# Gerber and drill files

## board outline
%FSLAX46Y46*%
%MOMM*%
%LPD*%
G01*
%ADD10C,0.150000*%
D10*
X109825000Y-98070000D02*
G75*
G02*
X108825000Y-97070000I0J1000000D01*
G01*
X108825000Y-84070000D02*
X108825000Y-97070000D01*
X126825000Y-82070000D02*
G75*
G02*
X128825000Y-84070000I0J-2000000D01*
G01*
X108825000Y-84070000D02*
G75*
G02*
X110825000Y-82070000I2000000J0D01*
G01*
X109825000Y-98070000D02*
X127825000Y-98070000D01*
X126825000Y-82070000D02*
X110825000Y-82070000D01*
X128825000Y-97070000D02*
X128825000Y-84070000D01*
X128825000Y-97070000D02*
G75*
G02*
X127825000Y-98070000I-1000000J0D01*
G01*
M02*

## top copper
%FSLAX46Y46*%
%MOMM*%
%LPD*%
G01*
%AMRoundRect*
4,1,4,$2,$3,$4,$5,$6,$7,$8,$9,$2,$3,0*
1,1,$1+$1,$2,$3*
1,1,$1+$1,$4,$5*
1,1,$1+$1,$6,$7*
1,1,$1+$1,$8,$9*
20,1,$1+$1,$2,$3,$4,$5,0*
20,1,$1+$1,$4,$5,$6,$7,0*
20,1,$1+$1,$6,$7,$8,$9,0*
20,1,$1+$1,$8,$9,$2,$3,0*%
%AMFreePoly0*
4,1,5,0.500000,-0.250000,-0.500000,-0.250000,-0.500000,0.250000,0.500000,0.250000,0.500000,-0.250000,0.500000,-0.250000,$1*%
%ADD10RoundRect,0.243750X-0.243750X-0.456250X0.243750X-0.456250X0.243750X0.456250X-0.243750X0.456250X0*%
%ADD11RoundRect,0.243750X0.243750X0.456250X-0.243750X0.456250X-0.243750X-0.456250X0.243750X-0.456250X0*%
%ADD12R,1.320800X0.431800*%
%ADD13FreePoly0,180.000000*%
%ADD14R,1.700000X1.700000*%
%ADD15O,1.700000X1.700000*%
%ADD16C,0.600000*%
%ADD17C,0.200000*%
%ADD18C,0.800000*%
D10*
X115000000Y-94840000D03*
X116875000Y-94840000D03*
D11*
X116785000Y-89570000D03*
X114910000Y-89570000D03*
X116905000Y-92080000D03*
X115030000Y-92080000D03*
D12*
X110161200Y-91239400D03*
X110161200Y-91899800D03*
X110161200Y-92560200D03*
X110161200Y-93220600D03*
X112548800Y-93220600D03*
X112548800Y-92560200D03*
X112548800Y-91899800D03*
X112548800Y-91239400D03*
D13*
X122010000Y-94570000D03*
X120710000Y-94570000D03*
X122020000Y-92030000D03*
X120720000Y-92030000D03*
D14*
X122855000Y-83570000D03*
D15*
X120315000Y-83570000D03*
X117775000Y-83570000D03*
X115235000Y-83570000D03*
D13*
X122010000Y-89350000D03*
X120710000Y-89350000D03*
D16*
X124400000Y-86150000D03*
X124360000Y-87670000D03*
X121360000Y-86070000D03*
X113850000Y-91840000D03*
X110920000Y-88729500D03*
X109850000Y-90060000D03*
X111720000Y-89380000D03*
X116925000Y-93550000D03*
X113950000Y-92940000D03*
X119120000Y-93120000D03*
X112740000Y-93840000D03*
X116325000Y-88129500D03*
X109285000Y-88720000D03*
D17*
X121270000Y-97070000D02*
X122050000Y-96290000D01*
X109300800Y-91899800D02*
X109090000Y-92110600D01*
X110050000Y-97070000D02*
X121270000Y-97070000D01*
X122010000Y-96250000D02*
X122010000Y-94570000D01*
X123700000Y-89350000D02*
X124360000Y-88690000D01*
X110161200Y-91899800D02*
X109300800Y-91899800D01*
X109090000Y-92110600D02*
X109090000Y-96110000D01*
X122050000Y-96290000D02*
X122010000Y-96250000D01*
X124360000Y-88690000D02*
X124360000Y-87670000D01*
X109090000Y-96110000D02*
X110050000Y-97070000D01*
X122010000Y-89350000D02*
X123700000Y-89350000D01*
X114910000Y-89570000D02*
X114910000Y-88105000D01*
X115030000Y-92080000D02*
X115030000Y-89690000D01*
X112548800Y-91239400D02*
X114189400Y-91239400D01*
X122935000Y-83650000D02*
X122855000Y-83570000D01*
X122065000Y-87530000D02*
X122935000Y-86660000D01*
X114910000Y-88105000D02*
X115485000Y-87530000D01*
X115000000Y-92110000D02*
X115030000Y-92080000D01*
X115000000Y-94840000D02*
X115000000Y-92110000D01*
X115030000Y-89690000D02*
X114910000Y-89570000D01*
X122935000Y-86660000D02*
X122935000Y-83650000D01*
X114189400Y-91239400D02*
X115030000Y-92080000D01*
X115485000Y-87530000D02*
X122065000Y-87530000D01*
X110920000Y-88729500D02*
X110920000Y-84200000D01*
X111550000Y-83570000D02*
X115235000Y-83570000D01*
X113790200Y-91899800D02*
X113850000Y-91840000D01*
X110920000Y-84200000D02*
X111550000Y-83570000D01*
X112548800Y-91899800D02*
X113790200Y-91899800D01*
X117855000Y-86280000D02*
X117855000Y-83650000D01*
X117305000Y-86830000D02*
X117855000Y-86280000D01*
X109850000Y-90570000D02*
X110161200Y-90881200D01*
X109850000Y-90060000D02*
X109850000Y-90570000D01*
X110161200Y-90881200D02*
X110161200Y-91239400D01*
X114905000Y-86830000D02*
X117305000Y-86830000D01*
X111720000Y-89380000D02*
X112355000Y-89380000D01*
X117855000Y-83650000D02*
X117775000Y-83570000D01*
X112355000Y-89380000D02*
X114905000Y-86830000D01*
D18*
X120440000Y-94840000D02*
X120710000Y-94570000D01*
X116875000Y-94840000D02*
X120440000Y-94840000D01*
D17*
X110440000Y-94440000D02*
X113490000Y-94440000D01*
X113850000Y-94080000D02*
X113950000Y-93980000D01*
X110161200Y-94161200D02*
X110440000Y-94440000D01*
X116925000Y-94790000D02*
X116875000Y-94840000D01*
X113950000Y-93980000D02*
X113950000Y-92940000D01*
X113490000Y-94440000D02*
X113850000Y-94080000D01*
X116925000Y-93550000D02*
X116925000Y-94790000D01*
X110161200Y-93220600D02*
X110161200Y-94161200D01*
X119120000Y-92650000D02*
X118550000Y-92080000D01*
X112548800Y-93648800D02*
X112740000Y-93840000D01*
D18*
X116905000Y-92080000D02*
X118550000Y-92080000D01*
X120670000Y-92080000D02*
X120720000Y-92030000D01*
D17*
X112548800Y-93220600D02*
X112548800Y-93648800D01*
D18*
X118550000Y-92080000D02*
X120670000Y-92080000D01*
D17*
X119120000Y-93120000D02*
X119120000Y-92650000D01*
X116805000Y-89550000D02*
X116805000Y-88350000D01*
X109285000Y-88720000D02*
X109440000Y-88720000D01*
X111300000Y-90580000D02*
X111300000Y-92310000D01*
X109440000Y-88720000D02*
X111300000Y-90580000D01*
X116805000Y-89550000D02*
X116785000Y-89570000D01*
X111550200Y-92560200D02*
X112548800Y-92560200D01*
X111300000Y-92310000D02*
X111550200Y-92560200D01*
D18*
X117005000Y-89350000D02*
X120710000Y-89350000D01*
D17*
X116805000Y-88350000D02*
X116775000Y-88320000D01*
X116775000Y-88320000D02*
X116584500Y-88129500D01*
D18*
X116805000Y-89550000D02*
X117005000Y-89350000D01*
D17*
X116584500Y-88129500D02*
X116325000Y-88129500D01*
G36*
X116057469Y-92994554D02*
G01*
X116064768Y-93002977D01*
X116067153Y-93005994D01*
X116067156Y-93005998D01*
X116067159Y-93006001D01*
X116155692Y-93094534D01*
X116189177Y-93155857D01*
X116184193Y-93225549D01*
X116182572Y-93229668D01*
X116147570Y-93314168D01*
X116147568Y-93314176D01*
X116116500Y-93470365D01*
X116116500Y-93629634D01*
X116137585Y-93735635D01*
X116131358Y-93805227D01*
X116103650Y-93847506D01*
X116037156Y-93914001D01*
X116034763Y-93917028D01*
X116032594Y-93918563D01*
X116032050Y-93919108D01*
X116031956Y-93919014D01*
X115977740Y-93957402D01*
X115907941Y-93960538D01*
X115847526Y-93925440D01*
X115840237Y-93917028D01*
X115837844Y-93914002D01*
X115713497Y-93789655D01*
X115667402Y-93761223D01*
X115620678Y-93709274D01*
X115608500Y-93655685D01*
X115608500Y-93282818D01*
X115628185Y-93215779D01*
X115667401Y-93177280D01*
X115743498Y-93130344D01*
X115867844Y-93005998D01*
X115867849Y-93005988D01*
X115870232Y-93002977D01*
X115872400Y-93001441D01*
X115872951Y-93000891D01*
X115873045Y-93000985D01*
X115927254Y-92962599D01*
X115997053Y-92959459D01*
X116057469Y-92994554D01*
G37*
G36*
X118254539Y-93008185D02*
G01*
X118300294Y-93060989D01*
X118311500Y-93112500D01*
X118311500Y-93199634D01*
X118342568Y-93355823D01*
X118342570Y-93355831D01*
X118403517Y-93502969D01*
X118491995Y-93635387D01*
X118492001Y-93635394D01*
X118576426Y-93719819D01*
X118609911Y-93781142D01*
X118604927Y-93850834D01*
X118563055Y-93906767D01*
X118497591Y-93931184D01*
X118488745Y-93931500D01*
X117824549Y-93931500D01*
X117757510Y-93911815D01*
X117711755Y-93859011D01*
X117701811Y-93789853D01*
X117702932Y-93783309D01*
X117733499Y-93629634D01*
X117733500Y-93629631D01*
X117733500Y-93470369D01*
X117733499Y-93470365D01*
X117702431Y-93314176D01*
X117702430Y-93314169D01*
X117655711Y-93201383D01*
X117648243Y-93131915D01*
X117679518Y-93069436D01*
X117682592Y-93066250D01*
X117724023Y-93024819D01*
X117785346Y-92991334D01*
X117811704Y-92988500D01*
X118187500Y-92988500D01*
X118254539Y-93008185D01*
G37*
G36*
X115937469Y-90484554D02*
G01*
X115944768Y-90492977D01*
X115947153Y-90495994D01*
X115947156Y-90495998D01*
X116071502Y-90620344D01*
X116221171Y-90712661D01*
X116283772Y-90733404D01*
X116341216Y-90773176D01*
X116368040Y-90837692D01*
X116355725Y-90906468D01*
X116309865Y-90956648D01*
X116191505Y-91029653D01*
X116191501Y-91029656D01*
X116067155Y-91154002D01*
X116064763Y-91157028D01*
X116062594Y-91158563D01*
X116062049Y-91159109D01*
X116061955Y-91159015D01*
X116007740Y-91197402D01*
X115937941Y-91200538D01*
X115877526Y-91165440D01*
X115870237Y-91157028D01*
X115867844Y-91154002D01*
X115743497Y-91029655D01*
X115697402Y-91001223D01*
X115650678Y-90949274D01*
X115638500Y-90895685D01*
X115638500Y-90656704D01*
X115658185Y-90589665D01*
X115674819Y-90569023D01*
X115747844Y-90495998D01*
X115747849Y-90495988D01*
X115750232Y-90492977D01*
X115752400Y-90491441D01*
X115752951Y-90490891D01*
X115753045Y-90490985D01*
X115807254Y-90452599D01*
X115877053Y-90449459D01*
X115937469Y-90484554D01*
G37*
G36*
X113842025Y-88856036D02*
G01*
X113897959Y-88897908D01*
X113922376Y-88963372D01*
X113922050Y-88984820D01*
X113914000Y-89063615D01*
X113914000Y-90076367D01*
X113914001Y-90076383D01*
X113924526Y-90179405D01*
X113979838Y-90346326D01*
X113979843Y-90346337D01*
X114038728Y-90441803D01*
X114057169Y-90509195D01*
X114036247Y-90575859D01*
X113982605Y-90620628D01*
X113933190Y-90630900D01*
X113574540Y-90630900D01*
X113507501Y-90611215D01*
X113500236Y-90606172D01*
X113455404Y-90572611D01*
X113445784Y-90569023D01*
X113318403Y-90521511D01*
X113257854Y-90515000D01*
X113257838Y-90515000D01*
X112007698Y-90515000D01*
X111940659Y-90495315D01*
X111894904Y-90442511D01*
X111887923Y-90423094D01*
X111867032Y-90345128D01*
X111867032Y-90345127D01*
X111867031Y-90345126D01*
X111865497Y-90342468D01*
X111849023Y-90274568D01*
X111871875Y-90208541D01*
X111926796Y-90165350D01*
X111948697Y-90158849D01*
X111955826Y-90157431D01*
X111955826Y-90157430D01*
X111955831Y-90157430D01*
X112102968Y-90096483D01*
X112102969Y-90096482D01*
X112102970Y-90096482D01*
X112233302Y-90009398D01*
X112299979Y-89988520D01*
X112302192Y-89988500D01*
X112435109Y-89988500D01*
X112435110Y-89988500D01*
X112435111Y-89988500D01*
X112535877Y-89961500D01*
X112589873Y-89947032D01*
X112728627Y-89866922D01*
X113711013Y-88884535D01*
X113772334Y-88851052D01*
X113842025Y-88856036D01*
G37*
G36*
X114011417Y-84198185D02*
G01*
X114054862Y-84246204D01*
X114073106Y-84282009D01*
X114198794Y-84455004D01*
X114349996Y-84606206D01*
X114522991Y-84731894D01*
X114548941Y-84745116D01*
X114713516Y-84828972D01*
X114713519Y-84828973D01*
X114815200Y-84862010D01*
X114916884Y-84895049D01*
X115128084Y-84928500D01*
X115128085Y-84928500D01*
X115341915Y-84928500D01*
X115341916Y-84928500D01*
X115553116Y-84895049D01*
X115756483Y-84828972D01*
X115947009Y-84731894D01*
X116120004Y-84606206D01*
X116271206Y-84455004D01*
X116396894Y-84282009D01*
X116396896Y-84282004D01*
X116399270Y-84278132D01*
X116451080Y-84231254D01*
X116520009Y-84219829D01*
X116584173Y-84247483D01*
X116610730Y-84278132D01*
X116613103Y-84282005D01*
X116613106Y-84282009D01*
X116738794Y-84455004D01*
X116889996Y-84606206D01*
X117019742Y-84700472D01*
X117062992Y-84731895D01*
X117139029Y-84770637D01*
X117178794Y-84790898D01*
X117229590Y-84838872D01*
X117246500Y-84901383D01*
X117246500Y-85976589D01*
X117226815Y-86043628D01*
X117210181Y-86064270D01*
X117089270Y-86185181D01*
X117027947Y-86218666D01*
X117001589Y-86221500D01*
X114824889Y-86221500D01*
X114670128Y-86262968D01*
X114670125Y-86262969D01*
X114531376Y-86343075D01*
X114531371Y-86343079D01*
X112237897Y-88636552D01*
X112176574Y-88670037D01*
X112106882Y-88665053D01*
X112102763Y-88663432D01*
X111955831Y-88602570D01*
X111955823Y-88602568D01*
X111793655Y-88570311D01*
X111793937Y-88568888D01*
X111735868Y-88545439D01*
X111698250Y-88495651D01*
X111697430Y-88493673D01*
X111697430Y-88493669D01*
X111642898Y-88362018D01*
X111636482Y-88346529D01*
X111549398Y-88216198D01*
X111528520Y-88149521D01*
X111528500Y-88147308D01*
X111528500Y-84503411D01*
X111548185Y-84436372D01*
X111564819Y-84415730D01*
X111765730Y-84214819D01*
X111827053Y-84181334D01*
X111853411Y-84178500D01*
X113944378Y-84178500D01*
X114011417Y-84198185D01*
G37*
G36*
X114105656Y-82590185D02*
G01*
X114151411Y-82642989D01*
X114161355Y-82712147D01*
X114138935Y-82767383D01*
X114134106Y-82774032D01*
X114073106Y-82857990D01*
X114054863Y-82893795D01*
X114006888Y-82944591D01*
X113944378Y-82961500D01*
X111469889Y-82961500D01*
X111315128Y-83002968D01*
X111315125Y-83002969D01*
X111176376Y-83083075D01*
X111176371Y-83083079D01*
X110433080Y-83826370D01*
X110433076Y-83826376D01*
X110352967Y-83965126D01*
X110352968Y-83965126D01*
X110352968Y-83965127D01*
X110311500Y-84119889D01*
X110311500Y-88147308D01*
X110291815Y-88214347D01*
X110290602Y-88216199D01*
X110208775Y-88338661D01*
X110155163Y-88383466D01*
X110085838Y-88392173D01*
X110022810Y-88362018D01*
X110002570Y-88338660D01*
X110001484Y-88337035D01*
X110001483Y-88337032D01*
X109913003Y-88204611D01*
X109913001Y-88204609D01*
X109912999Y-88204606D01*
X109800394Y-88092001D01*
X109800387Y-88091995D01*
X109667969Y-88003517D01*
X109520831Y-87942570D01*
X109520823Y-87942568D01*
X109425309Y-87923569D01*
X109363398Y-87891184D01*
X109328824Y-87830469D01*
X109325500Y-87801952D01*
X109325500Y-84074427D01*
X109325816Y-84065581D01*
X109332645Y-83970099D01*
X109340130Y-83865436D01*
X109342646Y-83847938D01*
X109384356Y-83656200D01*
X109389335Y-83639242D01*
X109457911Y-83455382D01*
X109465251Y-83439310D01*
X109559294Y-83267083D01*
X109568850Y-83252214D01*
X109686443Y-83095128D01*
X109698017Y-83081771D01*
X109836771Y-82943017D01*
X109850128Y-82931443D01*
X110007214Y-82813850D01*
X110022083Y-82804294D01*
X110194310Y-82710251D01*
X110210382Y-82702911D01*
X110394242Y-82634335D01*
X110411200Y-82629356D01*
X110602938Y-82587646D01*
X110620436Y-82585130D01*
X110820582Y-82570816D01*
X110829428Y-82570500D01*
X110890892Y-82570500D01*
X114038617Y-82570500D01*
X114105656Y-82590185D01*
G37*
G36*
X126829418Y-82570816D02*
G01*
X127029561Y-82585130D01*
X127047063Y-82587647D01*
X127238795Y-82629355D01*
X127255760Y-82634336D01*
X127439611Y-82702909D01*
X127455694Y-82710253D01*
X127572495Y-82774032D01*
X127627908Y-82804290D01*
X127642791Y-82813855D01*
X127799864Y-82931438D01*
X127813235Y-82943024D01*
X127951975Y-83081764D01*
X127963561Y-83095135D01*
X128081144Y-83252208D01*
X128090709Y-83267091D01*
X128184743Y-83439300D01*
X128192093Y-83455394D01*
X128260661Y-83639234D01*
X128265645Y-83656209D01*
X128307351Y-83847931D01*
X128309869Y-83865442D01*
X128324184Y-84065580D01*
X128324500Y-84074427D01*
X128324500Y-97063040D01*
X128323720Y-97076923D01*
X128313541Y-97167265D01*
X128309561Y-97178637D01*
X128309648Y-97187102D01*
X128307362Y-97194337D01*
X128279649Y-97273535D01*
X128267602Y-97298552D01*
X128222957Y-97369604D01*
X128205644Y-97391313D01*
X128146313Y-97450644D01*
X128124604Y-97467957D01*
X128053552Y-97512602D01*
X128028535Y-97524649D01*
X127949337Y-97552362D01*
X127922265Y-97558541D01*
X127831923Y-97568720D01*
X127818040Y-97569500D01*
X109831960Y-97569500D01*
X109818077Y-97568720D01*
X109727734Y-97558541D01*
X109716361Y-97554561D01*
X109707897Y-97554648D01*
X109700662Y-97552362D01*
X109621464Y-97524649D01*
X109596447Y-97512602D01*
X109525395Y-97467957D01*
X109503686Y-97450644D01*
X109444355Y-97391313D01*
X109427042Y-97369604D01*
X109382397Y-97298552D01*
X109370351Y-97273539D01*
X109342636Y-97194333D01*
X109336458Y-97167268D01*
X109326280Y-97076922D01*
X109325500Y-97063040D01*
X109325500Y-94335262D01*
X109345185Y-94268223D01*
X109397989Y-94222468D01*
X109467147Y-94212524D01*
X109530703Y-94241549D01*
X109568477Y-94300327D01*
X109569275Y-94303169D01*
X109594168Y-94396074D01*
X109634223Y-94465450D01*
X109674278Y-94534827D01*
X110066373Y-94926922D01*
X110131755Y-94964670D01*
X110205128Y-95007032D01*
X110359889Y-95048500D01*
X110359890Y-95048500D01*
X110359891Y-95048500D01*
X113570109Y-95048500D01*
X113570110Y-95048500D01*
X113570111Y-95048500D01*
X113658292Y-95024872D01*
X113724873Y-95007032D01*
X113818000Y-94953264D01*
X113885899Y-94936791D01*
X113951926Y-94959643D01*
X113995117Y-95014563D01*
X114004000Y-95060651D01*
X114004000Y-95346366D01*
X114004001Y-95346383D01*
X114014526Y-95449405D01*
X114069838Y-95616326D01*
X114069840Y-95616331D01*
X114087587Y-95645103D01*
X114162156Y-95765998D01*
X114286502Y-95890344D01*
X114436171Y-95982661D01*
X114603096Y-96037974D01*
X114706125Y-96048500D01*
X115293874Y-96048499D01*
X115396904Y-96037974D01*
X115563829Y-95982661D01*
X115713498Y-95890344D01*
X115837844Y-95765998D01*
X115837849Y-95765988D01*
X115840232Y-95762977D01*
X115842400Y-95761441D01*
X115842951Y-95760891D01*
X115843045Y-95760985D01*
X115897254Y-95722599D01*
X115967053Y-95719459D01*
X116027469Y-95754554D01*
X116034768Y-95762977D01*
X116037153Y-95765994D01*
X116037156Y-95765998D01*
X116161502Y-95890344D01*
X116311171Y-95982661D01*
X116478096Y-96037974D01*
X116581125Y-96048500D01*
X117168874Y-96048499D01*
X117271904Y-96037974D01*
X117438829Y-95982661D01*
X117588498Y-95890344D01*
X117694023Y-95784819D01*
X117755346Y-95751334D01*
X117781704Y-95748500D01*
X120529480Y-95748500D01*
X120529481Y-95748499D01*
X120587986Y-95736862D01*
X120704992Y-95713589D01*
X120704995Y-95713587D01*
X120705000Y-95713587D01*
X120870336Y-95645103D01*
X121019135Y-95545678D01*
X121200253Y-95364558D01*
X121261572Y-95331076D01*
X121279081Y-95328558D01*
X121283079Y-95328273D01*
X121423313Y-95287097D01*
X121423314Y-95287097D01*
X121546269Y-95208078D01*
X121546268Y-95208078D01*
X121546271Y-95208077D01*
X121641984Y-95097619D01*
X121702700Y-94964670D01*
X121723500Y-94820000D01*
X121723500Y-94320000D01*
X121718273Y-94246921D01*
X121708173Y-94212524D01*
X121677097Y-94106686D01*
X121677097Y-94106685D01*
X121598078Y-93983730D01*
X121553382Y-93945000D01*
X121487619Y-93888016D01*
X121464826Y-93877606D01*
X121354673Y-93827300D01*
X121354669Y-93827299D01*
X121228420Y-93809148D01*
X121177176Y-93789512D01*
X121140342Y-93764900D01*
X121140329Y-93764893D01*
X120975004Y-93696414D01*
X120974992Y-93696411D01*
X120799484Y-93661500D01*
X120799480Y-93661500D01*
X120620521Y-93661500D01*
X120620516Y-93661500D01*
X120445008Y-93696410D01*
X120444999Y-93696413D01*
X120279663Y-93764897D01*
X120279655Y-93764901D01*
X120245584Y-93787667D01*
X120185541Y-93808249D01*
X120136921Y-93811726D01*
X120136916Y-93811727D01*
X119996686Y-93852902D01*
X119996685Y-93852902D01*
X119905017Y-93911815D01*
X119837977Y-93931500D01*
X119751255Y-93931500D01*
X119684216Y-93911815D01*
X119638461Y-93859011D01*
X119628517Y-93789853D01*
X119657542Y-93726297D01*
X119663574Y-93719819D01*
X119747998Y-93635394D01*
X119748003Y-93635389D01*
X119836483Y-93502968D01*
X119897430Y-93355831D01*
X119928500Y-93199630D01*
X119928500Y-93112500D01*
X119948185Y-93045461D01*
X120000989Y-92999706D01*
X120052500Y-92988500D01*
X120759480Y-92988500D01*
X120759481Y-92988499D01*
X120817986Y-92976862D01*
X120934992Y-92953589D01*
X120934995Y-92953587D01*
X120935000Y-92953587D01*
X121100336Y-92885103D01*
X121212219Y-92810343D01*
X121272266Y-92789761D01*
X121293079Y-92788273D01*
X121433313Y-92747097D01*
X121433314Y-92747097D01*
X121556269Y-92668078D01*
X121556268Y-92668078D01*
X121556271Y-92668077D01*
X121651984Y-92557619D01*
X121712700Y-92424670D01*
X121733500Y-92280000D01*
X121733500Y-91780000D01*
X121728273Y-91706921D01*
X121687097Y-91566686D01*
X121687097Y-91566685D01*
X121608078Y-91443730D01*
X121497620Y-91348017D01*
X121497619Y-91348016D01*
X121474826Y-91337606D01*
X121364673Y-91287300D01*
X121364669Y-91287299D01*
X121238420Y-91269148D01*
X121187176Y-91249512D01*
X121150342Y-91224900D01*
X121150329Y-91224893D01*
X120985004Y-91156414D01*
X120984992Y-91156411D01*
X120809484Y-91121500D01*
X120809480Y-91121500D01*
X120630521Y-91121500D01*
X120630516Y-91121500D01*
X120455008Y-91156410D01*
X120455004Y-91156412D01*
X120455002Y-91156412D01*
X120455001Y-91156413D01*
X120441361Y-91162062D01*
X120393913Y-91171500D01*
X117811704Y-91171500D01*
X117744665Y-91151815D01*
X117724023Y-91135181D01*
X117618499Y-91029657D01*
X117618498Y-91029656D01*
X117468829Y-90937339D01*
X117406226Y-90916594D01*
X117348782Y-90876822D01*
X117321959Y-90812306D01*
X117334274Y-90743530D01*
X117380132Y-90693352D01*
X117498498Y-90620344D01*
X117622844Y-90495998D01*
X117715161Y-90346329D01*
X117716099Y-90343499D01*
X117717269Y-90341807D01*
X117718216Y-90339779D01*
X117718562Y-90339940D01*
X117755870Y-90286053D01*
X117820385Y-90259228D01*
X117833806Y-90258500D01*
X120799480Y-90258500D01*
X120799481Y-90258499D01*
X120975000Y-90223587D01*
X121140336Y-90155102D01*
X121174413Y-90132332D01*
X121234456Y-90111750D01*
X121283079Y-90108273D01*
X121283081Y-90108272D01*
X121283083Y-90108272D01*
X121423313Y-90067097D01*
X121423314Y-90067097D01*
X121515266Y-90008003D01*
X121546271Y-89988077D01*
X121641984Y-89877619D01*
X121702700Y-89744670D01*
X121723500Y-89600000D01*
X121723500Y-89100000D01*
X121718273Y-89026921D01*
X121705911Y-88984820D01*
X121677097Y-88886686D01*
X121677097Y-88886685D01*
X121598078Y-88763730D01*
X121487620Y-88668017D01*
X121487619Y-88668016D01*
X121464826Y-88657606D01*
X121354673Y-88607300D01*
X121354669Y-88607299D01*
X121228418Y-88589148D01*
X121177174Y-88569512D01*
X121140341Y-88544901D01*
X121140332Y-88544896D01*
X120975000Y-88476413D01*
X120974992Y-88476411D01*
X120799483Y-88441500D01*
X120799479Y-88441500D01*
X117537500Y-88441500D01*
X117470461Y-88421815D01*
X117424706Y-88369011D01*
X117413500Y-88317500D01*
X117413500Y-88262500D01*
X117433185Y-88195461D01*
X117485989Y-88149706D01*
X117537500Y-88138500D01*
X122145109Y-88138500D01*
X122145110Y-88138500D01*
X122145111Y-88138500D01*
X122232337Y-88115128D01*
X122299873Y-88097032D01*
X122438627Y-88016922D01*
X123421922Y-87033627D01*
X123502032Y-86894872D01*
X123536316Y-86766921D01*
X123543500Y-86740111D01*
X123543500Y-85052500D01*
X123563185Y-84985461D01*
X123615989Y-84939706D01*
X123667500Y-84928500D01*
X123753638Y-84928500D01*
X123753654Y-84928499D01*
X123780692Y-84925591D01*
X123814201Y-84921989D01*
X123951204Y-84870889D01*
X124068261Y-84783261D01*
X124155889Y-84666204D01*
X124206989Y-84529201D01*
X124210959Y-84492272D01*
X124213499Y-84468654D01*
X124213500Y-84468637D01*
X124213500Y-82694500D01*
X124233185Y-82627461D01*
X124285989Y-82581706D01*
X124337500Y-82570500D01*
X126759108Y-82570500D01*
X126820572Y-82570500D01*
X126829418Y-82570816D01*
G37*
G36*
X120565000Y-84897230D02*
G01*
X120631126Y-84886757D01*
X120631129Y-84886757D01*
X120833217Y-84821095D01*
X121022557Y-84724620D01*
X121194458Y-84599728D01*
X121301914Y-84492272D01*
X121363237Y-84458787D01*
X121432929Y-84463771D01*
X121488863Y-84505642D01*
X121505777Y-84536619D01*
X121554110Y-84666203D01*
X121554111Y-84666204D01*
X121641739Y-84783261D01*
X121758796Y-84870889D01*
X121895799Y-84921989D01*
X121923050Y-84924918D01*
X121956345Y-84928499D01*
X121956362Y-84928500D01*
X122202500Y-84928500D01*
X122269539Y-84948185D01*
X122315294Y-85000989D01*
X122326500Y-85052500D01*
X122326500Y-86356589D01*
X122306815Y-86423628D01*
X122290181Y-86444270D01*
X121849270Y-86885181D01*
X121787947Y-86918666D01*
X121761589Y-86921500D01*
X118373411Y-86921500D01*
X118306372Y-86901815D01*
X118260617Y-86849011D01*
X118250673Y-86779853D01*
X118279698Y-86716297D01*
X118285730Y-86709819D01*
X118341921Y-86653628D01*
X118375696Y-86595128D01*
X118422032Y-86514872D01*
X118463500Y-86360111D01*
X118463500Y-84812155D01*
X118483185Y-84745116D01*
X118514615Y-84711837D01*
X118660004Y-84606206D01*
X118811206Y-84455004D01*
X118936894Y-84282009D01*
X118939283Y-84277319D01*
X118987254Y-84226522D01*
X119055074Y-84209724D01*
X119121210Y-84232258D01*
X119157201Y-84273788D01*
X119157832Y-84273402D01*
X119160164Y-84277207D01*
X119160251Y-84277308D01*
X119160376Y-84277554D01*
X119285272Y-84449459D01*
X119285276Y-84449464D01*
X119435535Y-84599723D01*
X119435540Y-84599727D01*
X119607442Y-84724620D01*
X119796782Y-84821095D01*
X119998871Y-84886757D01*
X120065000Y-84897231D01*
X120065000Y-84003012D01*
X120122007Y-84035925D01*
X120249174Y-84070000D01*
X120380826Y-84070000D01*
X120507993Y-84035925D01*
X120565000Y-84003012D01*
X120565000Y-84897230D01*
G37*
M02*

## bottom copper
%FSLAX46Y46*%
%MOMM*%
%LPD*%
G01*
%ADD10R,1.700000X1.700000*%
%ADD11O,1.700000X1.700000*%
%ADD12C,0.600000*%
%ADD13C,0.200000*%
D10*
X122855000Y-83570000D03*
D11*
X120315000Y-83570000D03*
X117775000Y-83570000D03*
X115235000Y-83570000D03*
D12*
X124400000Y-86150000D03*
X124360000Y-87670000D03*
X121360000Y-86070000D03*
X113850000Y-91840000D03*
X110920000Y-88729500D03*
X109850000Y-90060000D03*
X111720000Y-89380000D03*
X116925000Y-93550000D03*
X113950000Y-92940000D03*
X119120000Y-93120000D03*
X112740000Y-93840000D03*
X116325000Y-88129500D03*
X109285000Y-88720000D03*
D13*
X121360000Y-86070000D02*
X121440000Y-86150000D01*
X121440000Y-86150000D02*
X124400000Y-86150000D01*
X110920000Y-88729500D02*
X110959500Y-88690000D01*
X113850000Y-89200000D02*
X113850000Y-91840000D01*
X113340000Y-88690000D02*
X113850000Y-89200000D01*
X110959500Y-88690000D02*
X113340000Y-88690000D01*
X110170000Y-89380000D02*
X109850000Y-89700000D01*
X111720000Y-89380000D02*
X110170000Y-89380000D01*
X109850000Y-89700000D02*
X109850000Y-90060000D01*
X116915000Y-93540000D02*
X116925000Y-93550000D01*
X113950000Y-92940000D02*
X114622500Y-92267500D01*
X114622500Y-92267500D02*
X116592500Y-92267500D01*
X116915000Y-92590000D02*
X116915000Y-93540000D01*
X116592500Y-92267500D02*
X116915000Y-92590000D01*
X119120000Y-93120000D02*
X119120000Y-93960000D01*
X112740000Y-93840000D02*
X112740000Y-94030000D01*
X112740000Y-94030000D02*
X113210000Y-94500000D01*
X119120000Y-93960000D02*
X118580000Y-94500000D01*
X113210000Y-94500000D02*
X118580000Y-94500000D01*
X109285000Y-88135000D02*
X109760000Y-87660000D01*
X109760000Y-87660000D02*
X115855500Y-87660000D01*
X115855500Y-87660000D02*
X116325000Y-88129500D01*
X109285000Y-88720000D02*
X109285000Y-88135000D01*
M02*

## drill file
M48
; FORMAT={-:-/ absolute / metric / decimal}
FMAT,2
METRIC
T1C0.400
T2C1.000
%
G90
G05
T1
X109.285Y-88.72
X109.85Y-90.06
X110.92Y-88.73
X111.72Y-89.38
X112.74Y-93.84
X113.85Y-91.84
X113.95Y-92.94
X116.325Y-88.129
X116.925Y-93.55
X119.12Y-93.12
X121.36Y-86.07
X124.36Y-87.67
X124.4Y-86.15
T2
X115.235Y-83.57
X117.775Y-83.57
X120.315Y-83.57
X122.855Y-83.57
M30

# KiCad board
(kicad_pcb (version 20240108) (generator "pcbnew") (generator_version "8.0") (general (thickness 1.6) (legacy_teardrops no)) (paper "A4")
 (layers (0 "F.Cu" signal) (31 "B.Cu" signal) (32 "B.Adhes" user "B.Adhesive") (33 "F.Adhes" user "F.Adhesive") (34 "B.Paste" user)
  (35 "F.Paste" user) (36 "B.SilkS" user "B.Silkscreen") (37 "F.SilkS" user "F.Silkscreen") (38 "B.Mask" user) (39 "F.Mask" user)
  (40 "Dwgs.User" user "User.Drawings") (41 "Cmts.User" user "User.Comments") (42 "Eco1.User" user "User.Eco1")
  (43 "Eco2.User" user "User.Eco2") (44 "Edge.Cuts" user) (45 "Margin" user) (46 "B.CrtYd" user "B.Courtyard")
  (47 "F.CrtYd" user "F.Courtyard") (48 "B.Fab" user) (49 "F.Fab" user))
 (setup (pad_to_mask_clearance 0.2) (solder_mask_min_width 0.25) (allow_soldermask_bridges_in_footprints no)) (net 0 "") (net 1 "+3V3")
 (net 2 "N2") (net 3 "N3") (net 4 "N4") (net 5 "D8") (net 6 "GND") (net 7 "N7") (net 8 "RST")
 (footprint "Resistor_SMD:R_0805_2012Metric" (layer "F.Cu") (at 115.9375 94.84)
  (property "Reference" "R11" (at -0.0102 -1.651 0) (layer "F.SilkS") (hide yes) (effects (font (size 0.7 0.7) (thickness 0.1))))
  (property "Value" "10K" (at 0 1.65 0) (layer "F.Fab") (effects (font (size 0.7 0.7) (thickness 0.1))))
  (pad "1" smd roundrect (at -0.9375 0) (size 0.975 1.4) (layers "F.Cu" "F.Paste" "F.Mask") (roundrect_rratio 0.25) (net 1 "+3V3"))
  (pad "2" smd roundrect (at 0.9375 0) (size 0.975 1.4) (layers "F.Cu" "F.Paste" "F.Mask") (roundrect_rratio 0.25) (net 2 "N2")))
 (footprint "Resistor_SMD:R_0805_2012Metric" (layer "F.Cu") (at 115.8475 89.57 180)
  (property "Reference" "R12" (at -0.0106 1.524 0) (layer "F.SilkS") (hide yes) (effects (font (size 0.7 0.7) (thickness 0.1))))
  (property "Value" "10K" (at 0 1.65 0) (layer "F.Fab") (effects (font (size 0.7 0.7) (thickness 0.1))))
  (pad "1" smd roundrect (at -0.9375 0 180) (size 0.975 1.4) (layers "F.Cu" "F.Paste" "F.Mask") (roundrect_rratio 0.25) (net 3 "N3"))
  (pad "2" smd roundrect (at 0.9375 0 180) (size 0.975 1.4) (layers "F.Cu" "F.Paste" "F.Mask") (roundrect_rratio 0.25) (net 1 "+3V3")))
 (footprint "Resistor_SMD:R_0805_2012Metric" (layer "F.Cu") (at 115.9675 92.08 180)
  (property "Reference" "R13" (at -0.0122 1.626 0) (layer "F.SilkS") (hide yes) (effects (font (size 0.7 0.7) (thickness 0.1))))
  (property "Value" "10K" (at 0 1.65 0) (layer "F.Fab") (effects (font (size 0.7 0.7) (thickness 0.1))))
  (pad "1" smd roundrect (at -0.9375 0 180) (size 0.975 1.4) (layers "F.Cu" "F.Paste" "F.Mask") (roundrect_rratio 0.25) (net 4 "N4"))
  (pad "2" smd roundrect (at 0.9375 0 180) (size 0.975 1.4) (layers "F.Cu" "F.Paste" "F.Mask") (roundrect_rratio 0.25) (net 1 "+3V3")))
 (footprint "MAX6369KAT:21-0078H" (layer "F.Cu") (at 111.355 92.23)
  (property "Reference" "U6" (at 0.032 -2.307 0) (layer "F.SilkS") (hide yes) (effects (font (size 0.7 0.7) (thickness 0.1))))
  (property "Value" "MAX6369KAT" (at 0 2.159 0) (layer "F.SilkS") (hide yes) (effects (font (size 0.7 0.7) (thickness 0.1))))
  (pad "1" smd rect (at -1.1938 -0.9906) (size 1.3208 0.4318) (layers "F.Cu" "F.Paste" "F.Mask") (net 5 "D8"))
  (pad "2" smd rect (at -1.1938 -0.3302) (size 1.3208 0.4318) (layers "F.Cu" "F.Paste" "F.Mask") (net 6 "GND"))
  (pad "3" smd rect (at -1.1938 0.3302) (size 1.3208 0.4318) (layers "F.Cu" "F.Paste" "F.Mask") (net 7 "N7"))
  (pad "4" smd rect (at -1.1938 0.9906) (size 1.3208 0.4318) (layers "F.Cu" "F.Paste" "F.Mask") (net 2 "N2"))
  (pad "5" smd rect (at 1.1938 0.9906) (size 1.3208 0.4318) (layers "F.Cu" "F.Paste" "F.Mask") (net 4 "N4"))
  (pad "6" smd rect (at 1.1938 0.3302) (size 1.3208 0.4318) (layers "F.Cu" "F.Paste" "F.Mask") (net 3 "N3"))
  (pad "7" smd rect (at 1.1938 -0.3302) (size 1.3208 0.4318) (layers "F.Cu" "F.Paste" "F.Mask") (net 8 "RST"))
  (pad "8" smd rect (at 1.1938 -0.9906) (size 1.3208 0.4318) (layers "F.Cu" "F.Paste" "F.Mask") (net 1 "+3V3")))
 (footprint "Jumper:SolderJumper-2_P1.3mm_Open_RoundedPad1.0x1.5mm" (layer "F.Cu") (at 121.36 94.57 180)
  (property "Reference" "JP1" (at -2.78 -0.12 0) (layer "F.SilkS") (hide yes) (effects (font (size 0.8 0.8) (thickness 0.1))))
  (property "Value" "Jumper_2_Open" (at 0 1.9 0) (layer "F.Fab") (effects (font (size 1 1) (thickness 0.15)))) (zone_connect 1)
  (pad "1" smd custom (at -0.65 0 180) (size 1 0.5) (layers "F.Cu" "F.Mask") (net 6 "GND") (zone_connect 2) (thermal_bridge_angle 45)
   (options (clearance outline) (anchor rect)) (primitives))
  (pad "2" smd custom (at 0.65 0 180) (size 1 0.5) (layers "F.Cu" "F.Mask") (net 2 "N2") (zone_connect 2) (thermal_bridge_angle 45)
   (options (clearance outline) (anchor rect)) (primitives)))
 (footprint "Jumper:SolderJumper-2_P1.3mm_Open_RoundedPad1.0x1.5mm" (layer "F.Cu") (at 121.37 92.03 180)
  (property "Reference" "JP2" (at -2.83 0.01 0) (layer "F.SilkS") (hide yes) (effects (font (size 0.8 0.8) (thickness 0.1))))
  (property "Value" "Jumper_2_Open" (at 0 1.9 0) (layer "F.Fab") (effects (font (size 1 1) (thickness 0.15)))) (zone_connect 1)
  (pad "1" smd custom (at -0.65 0 180) (size 1 0.5) (layers "F.Cu" "F.Mask") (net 6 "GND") (zone_connect 2) (thermal_bridge_angle 45)
   (options (clearance outline) (anchor rect)) (primitives))
  (pad "2" smd custom (at 0.65 0 180) (size 1 0.5) (layers "F.Cu" "F.Mask") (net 4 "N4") (zone_connect 2) (thermal_bridge_angle 45)
   (options (clearance outline) (anchor rect)) (primitives)))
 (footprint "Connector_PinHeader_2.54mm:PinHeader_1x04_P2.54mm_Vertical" (layer "F.Cu") (at 122.855 83.57 -90)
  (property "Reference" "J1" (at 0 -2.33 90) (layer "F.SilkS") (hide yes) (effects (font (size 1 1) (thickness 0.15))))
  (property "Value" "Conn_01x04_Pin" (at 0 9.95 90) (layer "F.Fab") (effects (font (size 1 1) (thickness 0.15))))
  (pad "1" thru_hole rect (at 0 0 270) (size 1.7 1.7) (drill 1) (layers "*.Cu" "*.Mask") (remove_unused_layers no) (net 1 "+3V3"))
  (pad "2" thru_hole oval (at 0 2.54 270) (size 1.7 1.7) (drill 1) (layers "*.Cu" "*.Mask") (remove_unused_layers no) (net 6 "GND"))
  (pad "3" thru_hole oval (at 0 5.08 270) (size 1.7 1.7) (drill 1) (layers "*.Cu" "*.Mask") (remove_unused_layers no) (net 5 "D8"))
  (pad "4" thru_hole oval (at 0 7.62 270) (size 1.7 1.7) (drill 1) (layers "*.Cu" "*.Mask") (remove_unused_layers no) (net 8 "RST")))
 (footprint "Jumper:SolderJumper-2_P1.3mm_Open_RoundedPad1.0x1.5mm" (layer "F.Cu") (at 121.36 89.35 180)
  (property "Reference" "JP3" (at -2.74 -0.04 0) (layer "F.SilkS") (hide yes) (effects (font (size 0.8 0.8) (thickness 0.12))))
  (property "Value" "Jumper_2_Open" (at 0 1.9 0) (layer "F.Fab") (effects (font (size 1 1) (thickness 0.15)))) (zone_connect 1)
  (pad "1" smd custom (at -0.65 0 180) (size 1 0.5) (layers "F.Cu" "F.Mask") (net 6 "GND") (zone_connect 2) (thermal_bridge_angle 45)
   (options (clearance outline) (anchor rect)) (primitives))
  (pad "2" smd custom (at 0.65 0 180) (size 1 0.5) (layers "F.Cu" "F.Mask") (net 3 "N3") (zone_connect 2) (thermal_bridge_angle 45)
   (options (clearance outline) (anchor rect)) (primitives)))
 (gr_arc (start 109.825 98.07) (mid 109.117893 97.777107) (end 108.825 97.07) (stroke (width 0.15) (type default)) (layer "Edge.Cuts"))
 (gr_line (start 108.825 84.07) (end 108.825 97.07) (stroke (width 0.15) (type default)) (layer "Edge.Cuts"))
 (gr_arc (start 126.825 82.07) (mid 128.239214 82.655786) (end 128.825 84.07) (stroke (width 0.15) (type default)) (layer "Edge.Cuts"))
 (gr_arc (start 108.825 84.07) (mid 109.410786 82.655786) (end 110.825 82.07) (stroke (width 0.15) (type default)) (layer "Edge.Cuts"))
 (gr_line (start 109.825 98.07) (end 127.825 98.07) (stroke (width 0.15) (type default)) (layer "Edge.Cuts"))
 (gr_line (start 126.825 82.07) (end 110.825 82.07) (stroke (width 0.15) (type default)) (layer "Edge.Cuts"))
 (gr_line (start 128.825 97.07) (end 128.825 84.07) (stroke (width 0.15) (type default)) (layer "Edge.Cuts"))
 (gr_arc (start 128.825 97.07) (mid 128.532107 97.777107) (end 127.825 98.07) (stroke (width 0.15) (type default)) (layer "Edge.Cuts"))
 (segment (start 121.27 97.07) (end 122.05 96.29) (width 0.2) (layer "F.Cu") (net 6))
 (segment (start 109.3008 91.8998) (end 109.09 92.1106) (width 0.2) (layer "F.Cu") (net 6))
 (segment (start 110.05 97.07) (end 121.27 97.07) (width 0.2) (layer "F.Cu") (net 6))
 (segment (start 122.01 96.25) (end 122.01 94.57) (width 0.2) (layer "F.Cu") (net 6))
 (segment (start 123.7 89.35) (end 124.36 88.69) (width 0.2) (layer "F.Cu") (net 6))
 (segment (start 110.1612 91.8998) (end 109.3008 91.8998) (width 0.2) (layer "F.Cu") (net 6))
 (segment (start 109.09 92.1106) (end 109.09 96.11) (width 0.2) (layer "F.Cu") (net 6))
 (segment (start 122.05 96.29) (end 122.01 96.25) (width 0.2) (layer "F.Cu") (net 6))
 (segment (start 124.36 88.69) (end 124.36 87.67) (width 0.2) (layer "F.Cu") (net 6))
 (segment (start 109.09 96.11) (end 110.05 97.07) (width 0.2) (layer "F.Cu") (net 6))
 (segment (start 122.01 89.35) (end 123.7 89.35) (width 0.2) (layer "F.Cu") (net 6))
 (via (at 124.4 86.15) (size 0.6) (drill 0.4) (layers "F.Cu" "B.Cu") (free yes) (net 6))
 (via (at 124.36 87.67) (size 0.6) (drill 0.4) (layers "F.Cu" "B.Cu") (free yes) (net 6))
 (via (at 121.36 86.07) (size 0.6) (drill 0.4) (layers "F.Cu" "B.Cu") (free yes) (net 6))
 (segment (start 121.36 86.07) (end 121.44 86.15) (width 0.2) (layer "B.Cu") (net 6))
 (segment (start 121.44 86.15) (end 124.4 86.15) (width 0.2) (layer "B.Cu") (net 6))
 (segment (start 114.91 89.57) (end 114.91 88.105) (width 0.2) (layer "F.Cu") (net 1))
 (segment (start 115.03 92.08) (end 115.03 89.69) (width 0.2) (layer "F.Cu") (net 1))
 (segment (start 112.5488 91.2394) (end 114.1894 91.2394) (width 0.2) (layer "F.Cu") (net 1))
 (segment (start 122.935 83.65) (end 122.855 83.57) (width 0.2) (layer "F.Cu") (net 1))
 (segment (start 122.065 87.53) (end 122.935 86.66) (width 0.2) (layer "F.Cu") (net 1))
 (segment (start 114.91 88.105) (end 115.485 87.53) (width 0.2) (layer "F.Cu") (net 1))
 (segment (start 115 92.11) (end 115.03 92.08) (width 0.2) (layer "F.Cu") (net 1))
 (segment (start 115 94.84) (end 115 92.11) (width 0.2) (layer "F.Cu") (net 1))
 (segment (start 115.03 89.69) (end 114.91 89.57) (width 0.2) (layer "F.Cu") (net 1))
 (segment (start 122.935 86.66) (end 122.935 83.65) (width 0.2) (layer "F.Cu") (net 1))
 (segment (start 114.1894 91.2394) (end 115.03 92.08) (width 0.2) (layer "F.Cu") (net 1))
 (segment (start 115.485 87.53) (end 122.065 87.53) (width 0.2) (layer "F.Cu") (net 1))
 (segment (start 110.92 88.7295) (end 110.92 84.2) (width 0.2) (layer "F.Cu") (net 8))
 (segment (start 111.55 83.57) (end 115.235 83.57) (width 0.2) (layer "F.Cu") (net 8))
 (segment (start 113.7902 91.8998) (end 113.85 91.84) (width 0.2) (layer "F.Cu") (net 8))
 (segment (start 110.92 84.2) (end 111.55 83.57) (width 0.2) (layer "F.Cu") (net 8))
 (segment (start 112.5488 91.8998) (end 113.7902 91.8998) (width 0.2) (layer "F.Cu") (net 8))
 (via (at 113.85 91.84) (size 0.6) (drill 0.4) (layers "F.Cu" "B.Cu") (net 8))
 (via (at 110.92 88.7295) (size 0.6) (drill 0.4) (layers "F.Cu" "B.Cu") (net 8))
 (segment (start 110.92 88.7295) (end 110.9595 88.69) (width 0.2) (layer "B.Cu") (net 8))
 (segment (start 113.85 89.2) (end 113.85 91.84) (width 0.2) (layer "B.Cu") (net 8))
 (segment (start 113.34 88.69) (end 113.85 89.2) (width 0.2) (layer "B.Cu") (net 8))
 (segment (start 110.9595 88.69) (end 113.34 88.69) (width 0.2) (layer "B.Cu") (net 8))
 (segment (start 117.855 86.28) (end 117.855 83.65) (width 0.2) (layer "F.Cu") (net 5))
 (segment (start 117.305 86.83) (end 117.855 86.28) (width 0.2) (layer "F.Cu") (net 5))
 (segment (start 109.85 90.57) (end 110.1612 90.8812) (width 0.2) (layer "F.Cu") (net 5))
 (segment (start 109.85 90.06) (end 109.85 90.57) (width 0.2) (layer "F.Cu") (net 5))
 (segment (start 110.1612 90.8812) (end 110.1612 91.2394) (width 0.2) (layer "F.Cu") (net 5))
 (segment (start 114.905 86.83) (end 117.305 86.83) (width 0.2) (layer "F.Cu") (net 5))
 (segment (start 111.72 89.38) (end 112.355 89.38) (width 0.2) (layer "F.Cu") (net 5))
 (segment (start 117.855 83.65) (end 117.775 83.57) (width 0.2) (layer "F.Cu") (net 5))
 (segment (start 112.355 89.38) (end 114.905 86.83) (width 0.2) (layer "F.Cu") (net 5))
 (via (at 109.85 90.06) (size 0.6) (drill 0.4) (layers "F.Cu" "B.Cu") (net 5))
 (via (at 111.72 89.38) (size 0.6) (drill 0.4) (layers "F.Cu" "B.Cu") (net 5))
 (segment (start 110.17 89.38) (end 109.85 89.7) (width 0.2) (layer "B.Cu") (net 5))
 (segment (start 111.72 89.38) (end 110.17 89.38) (width 0.2) (layer "B.Cu") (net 5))
 (segment (start 109.85 89.7) (end 109.85 90.06) (width 0.2) (layer "B.Cu") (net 5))
 (segment (start 120.44 94.84) (end 120.71 94.57) (width 0.8) (layer "F.Cu") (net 2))
 (segment (start 116.875 94.84) (end 120.44 94.84) (width 0.8) (layer "F.Cu") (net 2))
 (segment (start 110.44 94.44) (end 113.49 94.44) (width 0.2) (layer "F.Cu") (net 2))
 (segment (start 113.85 94.08) (end 113.95 93.98) (width 0.2) (layer "F.Cu") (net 2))
 (segment (start 110.1612 94.1612) (end 110.44 94.44) (width 0.2) (layer "F.Cu") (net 2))
 (segment (start 116.925 94.79) (end 116.875 94.84) (width 0.2) (layer "F.Cu") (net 2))
 (segment (start 113.95 93.98) (end 113.95 92.94) (width 0.2) (layer "F.Cu") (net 2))
 (segment (start 113.49 94.44) (end 113.85 94.08) (width 0.2) (layer "F.Cu") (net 2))
 (segment (start 116.925 93.55) (end 116.925 94.79) (width 0.2) (layer "F.Cu") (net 2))
 (segment (start 110.1612 93.2206) (end 110.1612 94.1612) (width 0.2) (layer "F.Cu") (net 2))
 (via (at 116.925 93.55) (size 0.6) (drill 0.4) (layers "F.Cu" "B.Cu") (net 2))
 (via (at 113.95 92.94) (size 0.6) (drill 0.4) (layers "F.Cu" "B.Cu") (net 2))
 (segment (start 116.915 93.54) (end 116.925 93.55) (width 0.2) (layer "B.Cu") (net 2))
 (segment (start 113.95 92.94) (end 114.6225 92.2675) (width 0.2) (layer "B.Cu") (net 2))
 (segment (start 114.6225 92.2675) (end 116.5925 92.2675) (width 0.2) (layer "B.Cu") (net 2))
 (segment (start 116.915 92.59) (end 116.915 93.54) (width 0.2) (layer "B.Cu") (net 2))
 (segment (start 116.5925 92.2675) (end 116.915 92.59) (width 0.2) (layer "B.Cu") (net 2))
 (segment (start 119.12 92.65) (end 118.55 92.08) (width 0.2) (layer "F.Cu") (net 4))
 (segment (start 112.5488 93.6488) (end 112.74 93.84) (width 0.2) (layer "F.Cu") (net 4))
 (segment (start 116.905 92.08) (end 118.55 92.08) (width 0.8) (layer "F.Cu") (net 4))
 (segment (start 120.67 92.08) (end 120.72 92.03) (width 0.8) (layer "F.Cu") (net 4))
 (segment (start 112.5488 93.2206) (end 112.5488 93.6488) (width 0.2) (layer "F.Cu") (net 4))
 (segment (start 118.55 92.08) (end 120.67 92.08) (width 0.8) (layer "F.Cu") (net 4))
 (segment (start 119.12 93.12) (end 119.12 92.65) (width 0.2) (layer "F.Cu") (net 4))
 (via (at 119.12 93.12) (size 0.6) (drill 0.4) (layers "F.Cu" "B.Cu") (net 4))
 (via (at 112.74 93.84) (size 0.6) (drill 0.4) (layers "F.Cu" "B.Cu") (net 4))
 (segment (start 119.12 93.12) (end 119.12 93.96) (width 0.2) (layer "B.Cu") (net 4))
 (segment (start 112.74 93.84) (end 112.74 94.03) (width 0.2) (layer "B.Cu") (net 4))
 (segment (start 112.74 94.03) (end 113.21 94.5) (width 0.2) (layer "B.Cu") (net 4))
 (segment (start 119.12 93.96) (end 118.58 94.5) (width 0.2) (layer "B.Cu") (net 4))
 (segment (start 113.21 94.5) (end 118.58 94.5) (width 0.2) (layer "B.Cu") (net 4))
 (segment (start 116.805 89.55) (end 116.805 88.35) (width 0.2) (layer "F.Cu") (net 3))
 (segment (start 109.285 88.72) (end 109.44 88.72) (width 0.2) (layer "F.Cu") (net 3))
 (segment (start 111.3 90.58) (end 111.3 92.31) (width 0.2) (layer "F.Cu") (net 3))
 (segment (start 109.44 88.72) (end 111.3 90.58) (width 0.2) (layer "F.Cu") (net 3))
 (segment (start 116.805 89.55) (end 116.785 89.57) (width 0.2) (layer "F.Cu") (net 3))
 (segment (start 111.5502 92.5602) (end 112.5488 92.5602) (width 0.2) (layer "F.Cu") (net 3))
 (segment (start 111.3 92.31) (end 111.5502 92.5602) (width 0.2) (layer "F.Cu") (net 3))
 (segment (start 117.005 89.35) (end 120.71 89.35) (width 0.8) (layer "F.Cu") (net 3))
 (segment (start 116.805 88.35) (end 116.775 88.32) (width 0.2) (layer "F.Cu") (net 3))
 (segment (start 116.775 88.32) (end 116.5845 88.1295) (width 0.2) (layer "F.Cu") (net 3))
 (segment (start 116.805 89.55) (end 117.005 89.35) (width 0.8) (layer "F.Cu") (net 3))
 (segment (start 116.5845 88.1295) (end 116.325 88.1295) (width 0.2) (layer "F.Cu") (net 3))
 (via (at 116.325 88.1295) (size 0.6) (drill 0.4) (layers "F.Cu" "B.Cu") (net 3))
 (via (at 109.285 88.72) (size 0.6) (drill 0.4) (layers "F.Cu" "B.Cu") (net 3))
 (segment (start 109.285 88.135) (end 109.76 87.66) (width 0.2) (layer "B.Cu") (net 3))
 (segment (start 109.76 87.66) (end 115.8555 87.66) (width 0.2) (layer "B.Cu") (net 3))
 (segment (start 115.8555 87.66) (end 116.325 88.1295) (width 0.2) (layer "B.Cu") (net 3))
 (segment (start 109.285 88.72) (end 109.285 88.135) (width 0.2) (layer "B.Cu") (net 3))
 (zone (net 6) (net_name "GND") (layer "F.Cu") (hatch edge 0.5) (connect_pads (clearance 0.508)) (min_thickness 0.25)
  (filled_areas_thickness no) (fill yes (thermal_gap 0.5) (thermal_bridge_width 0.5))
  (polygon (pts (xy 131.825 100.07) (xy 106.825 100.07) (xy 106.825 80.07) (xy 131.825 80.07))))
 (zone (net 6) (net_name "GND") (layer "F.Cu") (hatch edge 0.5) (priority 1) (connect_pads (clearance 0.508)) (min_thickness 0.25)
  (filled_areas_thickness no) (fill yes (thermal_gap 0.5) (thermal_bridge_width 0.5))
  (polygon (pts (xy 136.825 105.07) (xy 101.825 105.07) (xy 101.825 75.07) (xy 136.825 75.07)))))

